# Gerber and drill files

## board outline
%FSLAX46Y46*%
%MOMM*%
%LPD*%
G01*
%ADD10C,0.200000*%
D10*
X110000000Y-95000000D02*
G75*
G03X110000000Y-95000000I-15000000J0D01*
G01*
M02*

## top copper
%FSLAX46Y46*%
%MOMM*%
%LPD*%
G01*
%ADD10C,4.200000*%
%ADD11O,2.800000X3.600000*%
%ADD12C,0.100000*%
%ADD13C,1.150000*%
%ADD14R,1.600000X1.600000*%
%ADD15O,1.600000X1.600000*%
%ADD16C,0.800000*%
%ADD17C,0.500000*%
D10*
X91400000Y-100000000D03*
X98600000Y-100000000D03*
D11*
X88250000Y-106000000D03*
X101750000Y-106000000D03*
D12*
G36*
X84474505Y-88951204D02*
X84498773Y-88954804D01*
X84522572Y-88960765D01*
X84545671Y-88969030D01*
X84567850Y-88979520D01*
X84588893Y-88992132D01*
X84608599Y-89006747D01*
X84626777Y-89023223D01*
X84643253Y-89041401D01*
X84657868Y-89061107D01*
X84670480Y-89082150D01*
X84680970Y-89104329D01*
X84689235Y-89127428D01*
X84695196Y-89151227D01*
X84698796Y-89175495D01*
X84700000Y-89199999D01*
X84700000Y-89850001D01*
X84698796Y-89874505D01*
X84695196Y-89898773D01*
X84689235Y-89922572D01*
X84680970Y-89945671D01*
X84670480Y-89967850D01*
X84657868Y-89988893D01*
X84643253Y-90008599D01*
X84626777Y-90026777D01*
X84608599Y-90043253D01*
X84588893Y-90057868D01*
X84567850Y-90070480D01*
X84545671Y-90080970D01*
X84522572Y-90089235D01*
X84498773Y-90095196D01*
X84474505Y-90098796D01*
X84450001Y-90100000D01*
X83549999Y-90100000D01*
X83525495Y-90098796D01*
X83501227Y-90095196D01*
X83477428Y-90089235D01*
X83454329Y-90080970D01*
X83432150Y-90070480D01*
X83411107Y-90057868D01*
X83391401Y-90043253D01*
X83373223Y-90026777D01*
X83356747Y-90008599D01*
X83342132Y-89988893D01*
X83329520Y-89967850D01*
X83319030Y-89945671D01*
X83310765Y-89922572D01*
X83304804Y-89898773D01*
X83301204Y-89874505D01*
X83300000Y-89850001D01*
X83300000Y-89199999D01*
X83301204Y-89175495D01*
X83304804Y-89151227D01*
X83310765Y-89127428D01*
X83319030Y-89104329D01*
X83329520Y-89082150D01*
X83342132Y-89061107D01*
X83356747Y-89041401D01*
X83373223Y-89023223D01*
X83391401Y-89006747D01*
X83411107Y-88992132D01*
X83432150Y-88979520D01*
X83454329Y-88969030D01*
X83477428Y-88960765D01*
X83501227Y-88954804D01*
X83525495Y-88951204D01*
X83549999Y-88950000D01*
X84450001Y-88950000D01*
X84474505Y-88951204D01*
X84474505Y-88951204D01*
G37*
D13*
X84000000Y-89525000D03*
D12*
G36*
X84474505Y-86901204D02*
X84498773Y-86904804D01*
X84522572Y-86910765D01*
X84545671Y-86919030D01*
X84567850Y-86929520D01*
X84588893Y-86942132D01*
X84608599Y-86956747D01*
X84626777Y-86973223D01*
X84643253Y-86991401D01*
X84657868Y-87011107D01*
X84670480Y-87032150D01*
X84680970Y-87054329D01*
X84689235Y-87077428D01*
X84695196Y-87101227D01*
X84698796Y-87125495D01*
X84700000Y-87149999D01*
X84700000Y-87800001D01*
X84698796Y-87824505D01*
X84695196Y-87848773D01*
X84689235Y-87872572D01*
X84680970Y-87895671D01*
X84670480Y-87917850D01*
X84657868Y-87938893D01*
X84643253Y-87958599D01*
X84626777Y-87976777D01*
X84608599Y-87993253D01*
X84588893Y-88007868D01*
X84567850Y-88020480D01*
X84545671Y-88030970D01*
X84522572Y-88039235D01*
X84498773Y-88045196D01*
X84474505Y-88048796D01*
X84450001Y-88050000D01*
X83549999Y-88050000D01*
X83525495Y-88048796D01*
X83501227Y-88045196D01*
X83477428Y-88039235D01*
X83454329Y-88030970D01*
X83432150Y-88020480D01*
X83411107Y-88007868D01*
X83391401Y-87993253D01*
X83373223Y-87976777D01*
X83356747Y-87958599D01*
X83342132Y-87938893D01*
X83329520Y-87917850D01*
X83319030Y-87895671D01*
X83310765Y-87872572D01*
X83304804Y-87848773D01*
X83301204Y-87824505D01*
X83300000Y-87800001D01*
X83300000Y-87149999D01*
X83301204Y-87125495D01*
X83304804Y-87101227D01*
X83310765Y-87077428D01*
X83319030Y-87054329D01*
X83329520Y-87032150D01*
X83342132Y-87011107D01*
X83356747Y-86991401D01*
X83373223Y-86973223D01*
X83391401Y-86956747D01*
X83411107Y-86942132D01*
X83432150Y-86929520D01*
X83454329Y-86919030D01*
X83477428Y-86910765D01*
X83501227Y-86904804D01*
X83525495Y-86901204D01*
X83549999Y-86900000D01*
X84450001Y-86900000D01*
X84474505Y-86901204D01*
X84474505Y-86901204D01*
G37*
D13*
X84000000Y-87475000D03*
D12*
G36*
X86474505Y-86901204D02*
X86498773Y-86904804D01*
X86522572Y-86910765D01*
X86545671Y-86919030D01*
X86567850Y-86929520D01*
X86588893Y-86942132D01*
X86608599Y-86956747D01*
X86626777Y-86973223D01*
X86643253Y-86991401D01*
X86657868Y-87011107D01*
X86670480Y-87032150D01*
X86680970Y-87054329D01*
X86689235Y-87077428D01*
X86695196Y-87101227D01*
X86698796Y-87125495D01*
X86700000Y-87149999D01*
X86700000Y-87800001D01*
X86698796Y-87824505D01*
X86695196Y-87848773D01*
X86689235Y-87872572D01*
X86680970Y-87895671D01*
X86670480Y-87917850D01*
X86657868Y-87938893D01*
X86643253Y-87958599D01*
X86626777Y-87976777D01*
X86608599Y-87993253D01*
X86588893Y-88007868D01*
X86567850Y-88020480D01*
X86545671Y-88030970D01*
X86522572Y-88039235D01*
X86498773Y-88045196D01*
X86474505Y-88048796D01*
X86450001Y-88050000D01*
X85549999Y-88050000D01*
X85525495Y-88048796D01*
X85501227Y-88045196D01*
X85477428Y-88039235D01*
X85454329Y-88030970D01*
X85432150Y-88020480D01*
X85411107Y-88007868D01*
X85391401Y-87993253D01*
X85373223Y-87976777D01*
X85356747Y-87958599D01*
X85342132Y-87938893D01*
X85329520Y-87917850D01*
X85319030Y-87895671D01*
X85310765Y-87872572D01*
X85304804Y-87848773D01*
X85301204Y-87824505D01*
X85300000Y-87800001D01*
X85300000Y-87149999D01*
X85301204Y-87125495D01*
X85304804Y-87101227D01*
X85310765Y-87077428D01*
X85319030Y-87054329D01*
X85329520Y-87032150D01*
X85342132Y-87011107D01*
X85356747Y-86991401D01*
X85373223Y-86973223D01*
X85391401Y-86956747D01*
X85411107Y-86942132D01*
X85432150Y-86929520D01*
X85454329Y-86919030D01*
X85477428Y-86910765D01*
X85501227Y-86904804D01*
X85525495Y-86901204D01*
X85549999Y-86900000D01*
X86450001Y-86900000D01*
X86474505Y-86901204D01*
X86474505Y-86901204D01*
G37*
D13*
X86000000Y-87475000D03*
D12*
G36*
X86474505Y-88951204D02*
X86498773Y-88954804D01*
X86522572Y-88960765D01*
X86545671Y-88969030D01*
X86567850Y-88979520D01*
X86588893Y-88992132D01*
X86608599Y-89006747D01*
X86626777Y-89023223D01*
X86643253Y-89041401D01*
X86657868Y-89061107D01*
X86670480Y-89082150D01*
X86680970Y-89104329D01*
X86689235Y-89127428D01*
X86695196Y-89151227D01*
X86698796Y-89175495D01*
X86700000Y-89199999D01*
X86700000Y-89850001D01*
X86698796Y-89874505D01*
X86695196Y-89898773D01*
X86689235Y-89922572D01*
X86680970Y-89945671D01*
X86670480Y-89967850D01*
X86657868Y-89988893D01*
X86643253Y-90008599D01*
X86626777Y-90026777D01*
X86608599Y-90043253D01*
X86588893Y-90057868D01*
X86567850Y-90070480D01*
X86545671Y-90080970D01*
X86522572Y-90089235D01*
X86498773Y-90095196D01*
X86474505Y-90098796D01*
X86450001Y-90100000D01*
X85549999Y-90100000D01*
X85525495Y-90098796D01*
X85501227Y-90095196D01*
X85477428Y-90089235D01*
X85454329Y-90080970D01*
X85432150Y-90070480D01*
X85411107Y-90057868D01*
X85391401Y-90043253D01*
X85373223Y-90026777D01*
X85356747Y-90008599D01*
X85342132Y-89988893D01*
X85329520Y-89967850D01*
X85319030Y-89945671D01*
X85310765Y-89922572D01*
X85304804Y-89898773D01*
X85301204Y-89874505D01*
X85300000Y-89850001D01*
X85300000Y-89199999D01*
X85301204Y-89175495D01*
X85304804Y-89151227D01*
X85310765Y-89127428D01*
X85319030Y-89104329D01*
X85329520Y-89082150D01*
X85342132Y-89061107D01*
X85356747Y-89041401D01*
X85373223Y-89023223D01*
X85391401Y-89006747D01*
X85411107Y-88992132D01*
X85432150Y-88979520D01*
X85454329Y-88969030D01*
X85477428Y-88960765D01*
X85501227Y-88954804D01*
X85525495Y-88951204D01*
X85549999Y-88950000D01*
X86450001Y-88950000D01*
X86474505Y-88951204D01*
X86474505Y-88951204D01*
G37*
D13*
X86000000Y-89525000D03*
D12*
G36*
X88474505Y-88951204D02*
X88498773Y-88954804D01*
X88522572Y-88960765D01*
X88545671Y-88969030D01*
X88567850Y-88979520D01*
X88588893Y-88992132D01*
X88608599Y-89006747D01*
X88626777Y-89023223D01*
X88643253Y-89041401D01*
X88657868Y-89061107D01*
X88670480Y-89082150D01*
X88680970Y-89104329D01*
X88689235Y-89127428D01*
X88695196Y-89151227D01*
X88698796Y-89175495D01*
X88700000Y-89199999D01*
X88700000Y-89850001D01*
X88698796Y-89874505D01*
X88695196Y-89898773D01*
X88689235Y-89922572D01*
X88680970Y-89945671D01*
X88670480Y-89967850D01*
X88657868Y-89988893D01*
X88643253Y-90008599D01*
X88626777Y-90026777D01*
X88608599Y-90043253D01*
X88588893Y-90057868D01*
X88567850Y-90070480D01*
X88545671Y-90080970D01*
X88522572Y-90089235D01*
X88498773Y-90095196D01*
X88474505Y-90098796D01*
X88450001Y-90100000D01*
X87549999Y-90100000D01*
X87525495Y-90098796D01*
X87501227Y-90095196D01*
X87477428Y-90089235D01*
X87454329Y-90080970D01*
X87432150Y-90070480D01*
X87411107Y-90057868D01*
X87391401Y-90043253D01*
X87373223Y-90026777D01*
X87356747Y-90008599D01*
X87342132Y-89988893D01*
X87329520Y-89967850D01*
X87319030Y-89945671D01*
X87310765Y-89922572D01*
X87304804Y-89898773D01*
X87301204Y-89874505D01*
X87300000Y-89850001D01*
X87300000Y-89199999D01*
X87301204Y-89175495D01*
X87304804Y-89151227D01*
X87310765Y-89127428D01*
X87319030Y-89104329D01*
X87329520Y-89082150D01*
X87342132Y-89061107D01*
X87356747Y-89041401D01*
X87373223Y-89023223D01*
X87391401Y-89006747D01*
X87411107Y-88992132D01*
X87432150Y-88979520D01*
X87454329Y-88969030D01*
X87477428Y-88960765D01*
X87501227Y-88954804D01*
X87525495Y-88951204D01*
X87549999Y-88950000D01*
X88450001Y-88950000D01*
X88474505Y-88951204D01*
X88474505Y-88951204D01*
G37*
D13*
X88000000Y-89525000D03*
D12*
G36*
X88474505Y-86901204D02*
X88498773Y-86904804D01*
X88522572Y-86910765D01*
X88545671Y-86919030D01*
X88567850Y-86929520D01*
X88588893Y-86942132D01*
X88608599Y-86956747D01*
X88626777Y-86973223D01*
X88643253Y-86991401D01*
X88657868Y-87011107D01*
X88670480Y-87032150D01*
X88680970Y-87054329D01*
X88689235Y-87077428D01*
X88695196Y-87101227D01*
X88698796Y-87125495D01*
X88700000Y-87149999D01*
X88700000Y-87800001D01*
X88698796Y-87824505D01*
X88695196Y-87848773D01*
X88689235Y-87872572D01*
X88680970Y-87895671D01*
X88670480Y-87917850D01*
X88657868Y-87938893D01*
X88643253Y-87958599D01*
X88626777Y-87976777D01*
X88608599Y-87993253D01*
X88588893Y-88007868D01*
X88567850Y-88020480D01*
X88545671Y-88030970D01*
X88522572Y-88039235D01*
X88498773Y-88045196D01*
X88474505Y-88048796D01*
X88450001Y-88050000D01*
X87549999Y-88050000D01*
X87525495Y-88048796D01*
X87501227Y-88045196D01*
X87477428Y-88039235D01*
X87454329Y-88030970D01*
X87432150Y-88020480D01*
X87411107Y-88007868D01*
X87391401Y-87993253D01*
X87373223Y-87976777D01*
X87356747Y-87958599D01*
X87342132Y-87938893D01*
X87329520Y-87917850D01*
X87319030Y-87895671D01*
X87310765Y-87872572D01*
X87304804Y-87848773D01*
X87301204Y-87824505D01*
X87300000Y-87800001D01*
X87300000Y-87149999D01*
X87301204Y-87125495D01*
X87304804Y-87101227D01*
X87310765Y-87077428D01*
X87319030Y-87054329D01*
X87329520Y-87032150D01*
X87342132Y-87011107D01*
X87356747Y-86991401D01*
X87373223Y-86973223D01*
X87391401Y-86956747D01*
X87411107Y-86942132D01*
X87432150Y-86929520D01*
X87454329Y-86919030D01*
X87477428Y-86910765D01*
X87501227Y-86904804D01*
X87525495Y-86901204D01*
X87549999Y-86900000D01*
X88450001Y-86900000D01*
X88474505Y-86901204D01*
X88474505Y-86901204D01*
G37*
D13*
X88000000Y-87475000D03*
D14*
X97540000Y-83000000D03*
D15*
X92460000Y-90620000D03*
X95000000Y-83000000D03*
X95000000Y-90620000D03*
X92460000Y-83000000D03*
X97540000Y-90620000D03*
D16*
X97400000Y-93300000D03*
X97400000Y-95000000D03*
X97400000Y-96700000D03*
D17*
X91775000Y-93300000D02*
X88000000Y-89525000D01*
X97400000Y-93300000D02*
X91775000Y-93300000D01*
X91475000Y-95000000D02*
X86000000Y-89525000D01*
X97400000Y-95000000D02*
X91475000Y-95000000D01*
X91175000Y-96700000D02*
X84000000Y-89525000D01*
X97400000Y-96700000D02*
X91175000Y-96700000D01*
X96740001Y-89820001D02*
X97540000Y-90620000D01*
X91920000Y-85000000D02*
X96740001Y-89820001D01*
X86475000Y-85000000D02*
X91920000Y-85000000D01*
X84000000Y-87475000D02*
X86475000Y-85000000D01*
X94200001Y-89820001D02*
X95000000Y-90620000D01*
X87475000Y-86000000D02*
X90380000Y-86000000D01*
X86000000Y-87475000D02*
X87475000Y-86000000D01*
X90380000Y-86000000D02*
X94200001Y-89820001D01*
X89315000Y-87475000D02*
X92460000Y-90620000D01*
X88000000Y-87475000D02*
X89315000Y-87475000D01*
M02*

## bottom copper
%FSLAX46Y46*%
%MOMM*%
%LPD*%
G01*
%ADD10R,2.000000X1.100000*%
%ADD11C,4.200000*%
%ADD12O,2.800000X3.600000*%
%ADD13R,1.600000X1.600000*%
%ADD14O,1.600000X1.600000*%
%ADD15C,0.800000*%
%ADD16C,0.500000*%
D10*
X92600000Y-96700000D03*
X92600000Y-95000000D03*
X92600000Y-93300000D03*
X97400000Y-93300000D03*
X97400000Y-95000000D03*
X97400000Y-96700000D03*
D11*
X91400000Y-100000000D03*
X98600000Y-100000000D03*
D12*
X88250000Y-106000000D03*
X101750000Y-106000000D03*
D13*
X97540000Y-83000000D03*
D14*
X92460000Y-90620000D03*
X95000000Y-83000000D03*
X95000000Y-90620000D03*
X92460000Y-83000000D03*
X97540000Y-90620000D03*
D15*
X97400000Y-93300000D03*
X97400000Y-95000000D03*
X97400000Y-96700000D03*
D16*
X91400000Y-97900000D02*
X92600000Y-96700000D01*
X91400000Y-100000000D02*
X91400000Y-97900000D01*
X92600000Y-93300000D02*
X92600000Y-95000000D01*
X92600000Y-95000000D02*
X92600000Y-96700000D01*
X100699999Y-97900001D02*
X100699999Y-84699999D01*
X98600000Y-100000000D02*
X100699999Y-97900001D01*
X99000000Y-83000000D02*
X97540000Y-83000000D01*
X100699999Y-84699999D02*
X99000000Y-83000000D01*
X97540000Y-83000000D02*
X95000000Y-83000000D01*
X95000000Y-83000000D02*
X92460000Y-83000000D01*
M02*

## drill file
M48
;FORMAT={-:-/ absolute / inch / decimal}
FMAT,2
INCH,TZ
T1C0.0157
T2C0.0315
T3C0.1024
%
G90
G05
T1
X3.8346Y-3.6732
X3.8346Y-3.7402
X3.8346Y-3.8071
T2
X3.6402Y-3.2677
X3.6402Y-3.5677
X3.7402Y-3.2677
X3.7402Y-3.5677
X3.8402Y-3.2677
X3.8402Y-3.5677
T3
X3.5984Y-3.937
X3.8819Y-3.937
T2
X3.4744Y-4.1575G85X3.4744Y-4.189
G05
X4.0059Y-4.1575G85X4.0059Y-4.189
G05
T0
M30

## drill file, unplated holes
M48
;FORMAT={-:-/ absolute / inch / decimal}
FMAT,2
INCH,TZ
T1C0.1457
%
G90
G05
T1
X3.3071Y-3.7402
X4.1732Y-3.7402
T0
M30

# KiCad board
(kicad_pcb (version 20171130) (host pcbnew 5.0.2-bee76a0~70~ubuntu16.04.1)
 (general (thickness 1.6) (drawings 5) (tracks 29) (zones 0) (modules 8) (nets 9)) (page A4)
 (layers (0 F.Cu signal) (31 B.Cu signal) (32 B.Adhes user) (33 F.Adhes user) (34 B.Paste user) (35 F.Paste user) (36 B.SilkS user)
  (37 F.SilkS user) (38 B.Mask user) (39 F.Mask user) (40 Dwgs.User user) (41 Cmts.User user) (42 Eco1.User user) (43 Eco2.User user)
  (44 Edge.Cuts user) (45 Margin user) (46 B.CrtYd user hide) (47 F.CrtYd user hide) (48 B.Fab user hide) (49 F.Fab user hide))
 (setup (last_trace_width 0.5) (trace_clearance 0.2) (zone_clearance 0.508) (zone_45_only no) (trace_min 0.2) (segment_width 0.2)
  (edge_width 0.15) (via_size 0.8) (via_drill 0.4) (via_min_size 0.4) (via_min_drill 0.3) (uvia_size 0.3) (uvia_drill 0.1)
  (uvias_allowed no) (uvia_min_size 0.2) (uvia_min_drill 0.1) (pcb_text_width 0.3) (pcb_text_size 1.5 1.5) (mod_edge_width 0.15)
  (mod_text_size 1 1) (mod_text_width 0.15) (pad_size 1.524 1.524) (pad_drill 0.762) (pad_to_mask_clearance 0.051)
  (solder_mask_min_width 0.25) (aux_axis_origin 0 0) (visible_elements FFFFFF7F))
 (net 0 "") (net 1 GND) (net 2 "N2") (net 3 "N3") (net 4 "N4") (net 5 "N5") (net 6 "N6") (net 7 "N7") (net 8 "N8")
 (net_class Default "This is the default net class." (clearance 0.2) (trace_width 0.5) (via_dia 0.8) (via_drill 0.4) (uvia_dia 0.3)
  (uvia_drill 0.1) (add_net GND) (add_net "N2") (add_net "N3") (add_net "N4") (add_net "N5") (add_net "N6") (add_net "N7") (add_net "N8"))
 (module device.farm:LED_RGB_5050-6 (layer B.Cu) (at 95 95)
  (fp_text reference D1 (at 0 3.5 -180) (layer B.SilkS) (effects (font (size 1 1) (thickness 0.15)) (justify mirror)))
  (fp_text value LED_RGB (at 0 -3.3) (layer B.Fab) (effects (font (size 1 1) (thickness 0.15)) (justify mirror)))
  (pad 1 smd rect (at -2.4 1.7 270) (size 1.1 2) (layers B.Cu B.Paste B.Mask) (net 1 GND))
  (pad 2 smd rect (at -2.4 0 270) (size 1.1 2) (layers B.Cu B.Paste B.Mask) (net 1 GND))
  (pad 3 smd rect (at -2.4 -1.7 270) (size 1.1 2) (layers B.Cu B.Paste B.Mask) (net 1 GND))
  (pad 4 smd rect (at 2.4 -1.7 270) (size 1.1 2) (layers B.Cu B.Paste B.Mask) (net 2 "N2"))
  (pad 5 smd rect (at 2.4 0 270) (size 1.1 2) (layers B.Cu B.Paste B.Mask) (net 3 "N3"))
  (pad 6 smd rect (at 2.4 1.7 270) (size 1.1 2) (layers B.Cu B.Paste B.Mask) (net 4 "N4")))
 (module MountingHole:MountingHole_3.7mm (layer F.Cu) (at 84 95)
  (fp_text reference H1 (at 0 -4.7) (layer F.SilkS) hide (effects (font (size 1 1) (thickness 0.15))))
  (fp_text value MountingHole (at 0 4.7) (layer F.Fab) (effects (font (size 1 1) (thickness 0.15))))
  (pad 1 np_thru_hole circle (at 0 0) (size 3.7 3.7) (drill 3.7) (layers *.Cu *.Mask)))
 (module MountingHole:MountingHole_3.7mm (layer F.Cu) (at 106 95)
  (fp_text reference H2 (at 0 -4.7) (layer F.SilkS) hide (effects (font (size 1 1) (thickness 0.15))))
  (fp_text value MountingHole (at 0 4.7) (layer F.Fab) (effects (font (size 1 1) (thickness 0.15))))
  (pad 1 np_thru_hole circle (at 0 0) (size 3.7 3.7) (drill 3.7) (layers *.Cu *.Mask)))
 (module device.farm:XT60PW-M (layer F.Cu) (at 95 100)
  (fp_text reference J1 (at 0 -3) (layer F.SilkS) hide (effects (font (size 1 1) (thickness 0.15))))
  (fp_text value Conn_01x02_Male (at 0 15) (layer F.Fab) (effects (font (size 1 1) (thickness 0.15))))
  (pad 1 thru_hole circle (at -3.6 0) (size 4.2 4.2) (drill 2.6) (layers *.Cu *.Mask) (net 1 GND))
  (pad 2 thru_hole circle (at 3.6 0) (size 4.2 4.2) (drill 2.6) (layers *.Cu *.Mask) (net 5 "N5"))
  (pad "" thru_hole oval (at -6.75 6) (size 2.8 3.6) (drill oval 0.8 1.6) (layers *.Cu *.Mask))
  (pad "" thru_hole oval (at 6.75 6) (size 2.8 3.6) (drill oval 0.8 1.6) (layers *.Cu *.Mask)))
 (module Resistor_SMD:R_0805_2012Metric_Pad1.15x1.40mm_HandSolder (layer F.Cu) (at 84 88.5 90)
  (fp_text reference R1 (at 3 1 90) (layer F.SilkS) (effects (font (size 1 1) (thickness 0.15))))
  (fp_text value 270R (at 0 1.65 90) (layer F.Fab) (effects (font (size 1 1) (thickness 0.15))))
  (pad 1 smd roundrect (at -1.025 0 90) (size 1.15 1.4) (layers F.Cu F.Paste F.Mask) (roundrect_rratio 0.217391) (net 4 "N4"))
  (pad 2 smd roundrect (at 1.025 0 90) (size 1.15 1.4) (layers F.Cu F.Paste F.Mask) (roundrect_rratio 0.217391) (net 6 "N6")))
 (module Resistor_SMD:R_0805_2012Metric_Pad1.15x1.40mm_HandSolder (layer F.Cu) (at 86 88.5 90)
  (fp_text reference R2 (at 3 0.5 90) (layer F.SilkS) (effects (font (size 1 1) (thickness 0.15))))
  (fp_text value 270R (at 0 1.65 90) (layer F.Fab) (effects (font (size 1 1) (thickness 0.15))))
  (pad 2 smd roundrect (at 1.025 0 90) (size 1.15 1.4) (layers F.Cu F.Paste F.Mask) (roundrect_rratio 0.217391) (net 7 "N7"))
  (pad 1 smd roundrect (at -1.025 0 90) (size 1.15 1.4) (layers F.Cu F.Paste F.Mask) (roundrect_rratio 0.217391) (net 3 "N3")))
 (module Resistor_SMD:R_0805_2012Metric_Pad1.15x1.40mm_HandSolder (layer F.Cu) (at 88 88.5 90)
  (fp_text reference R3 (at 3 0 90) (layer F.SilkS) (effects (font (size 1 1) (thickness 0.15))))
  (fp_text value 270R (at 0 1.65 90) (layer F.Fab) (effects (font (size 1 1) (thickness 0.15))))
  (pad 1 smd roundrect (at -1.025 0 90) (size 1.15 1.4) (layers F.Cu F.Paste F.Mask) (roundrect_rratio 0.217391) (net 2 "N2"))
  (pad 2 smd roundrect (at 1.025 0 90) (size 1.15 1.4) (layers F.Cu F.Paste F.Mask) (roundrect_rratio 0.217391) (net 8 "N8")))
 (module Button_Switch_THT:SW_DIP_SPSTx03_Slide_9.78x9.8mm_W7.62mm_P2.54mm (layer F.Cu) (at 97.54 83 270)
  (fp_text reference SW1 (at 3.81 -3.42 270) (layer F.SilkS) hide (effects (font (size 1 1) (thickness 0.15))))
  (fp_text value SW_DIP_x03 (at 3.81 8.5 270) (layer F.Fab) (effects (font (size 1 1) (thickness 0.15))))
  (pad 1 thru_hole rect (at 0 0 270) (size 1.6 1.6) (drill 0.8) (layers *.Cu *.Mask) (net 5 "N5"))
  (pad 4 thru_hole oval (at 7.62 5.08 270) (size 1.6 1.6) (drill 0.8) (layers *.Cu *.Mask) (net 8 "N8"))
  (pad 2 thru_hole oval (at 0 2.54 270) (size 1.6 1.6) (drill 0.8) (layers *.Cu *.Mask) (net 5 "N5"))
  (pad 5 thru_hole oval (at 7.62 2.54 270) (size 1.6 1.6) (drill 0.8) (layers *.Cu *.Mask) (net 7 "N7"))
  (pad 3 thru_hole oval (at 0 5.08 270) (size 1.6 1.6) (drill 0.8) (layers *.Cu *.Mask) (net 5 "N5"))
  (pad 6 thru_hole oval (at 7.62 0 270) (size 1.6 1.6) (drill 0.8) (layers *.Cu *.Mask) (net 6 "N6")))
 (gr_circle (center 95 95) (end 110 95) (layer Edge.Cuts) (width 0.2))
 (segment (start 91.4 97.9) (end 92.6 96.7) (width 0.5) (layer B.Cu) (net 1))
 (segment (start 91.4 100) (end 91.4 97.9) (width 0.5) (layer B.Cu) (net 1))
 (segment (start 92.6 93.3) (end 92.6 95) (width 0.5) (layer B.Cu) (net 1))
 (segment (start 92.6 95) (end 92.6 96.7) (width 0.5) (layer B.Cu) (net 1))
 (via (at 97.4 93.3) (size 0.8) (drill 0.4) (layers F.Cu B.Cu) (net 2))
 (segment (start 91.775 93.3) (end 88 89.525) (width 0.5) (layer F.Cu) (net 2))
 (segment (start 97.4 93.3) (end 91.775 93.3) (width 0.5) (layer F.Cu) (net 2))
 (via (at 97.4 95) (size 0.8) (drill 0.4) (layers F.Cu B.Cu) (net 3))
 (segment (start 91.475 95) (end 86 89.525) (width 0.5) (layer F.Cu) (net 3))
 (segment (start 97.4 95) (end 91.475 95) (width 0.5) (layer F.Cu) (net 3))
 (via (at 97.4 96.7) (size 0.8) (drill 0.4) (layers F.Cu B.Cu) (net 4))
 (segment (start 91.175 96.7) (end 84 89.525) (width 0.5) (layer F.Cu) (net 4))
 (segment (start 97.4 96.7) (end 91.175 96.7) (width 0.5) (layer F.Cu) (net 4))
 (segment (start 100.699999 97.900001) (end 100.699999 84.699999) (width 0.5) (layer B.Cu) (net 5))
 (segment (start 98.6 100) (end 100.699999 97.900001) (width 0.5) (layer B.Cu) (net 5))
 (segment (start 99 83) (end 97.54 83) (width 0.5) (layer B.Cu) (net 5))
 (segment (start 100.699999 84.699999) (end 99 83) (width 0.5) (layer B.Cu) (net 5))
 (segment (start 97.54 83) (end 95 83) (width 0.5) (layer B.Cu) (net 5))
 (segment (start 95 83) (end 92.46 83) (width 0.5) (layer B.Cu) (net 5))
 (segment (start 96.740001 89.820001) (end 97.54 90.62) (width 0.5) (layer F.Cu) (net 6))
 (segment (start 91.92 85) (end 96.740001 89.820001) (width 0.5) (layer F.Cu) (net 6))
 (segment (start 86.475 85) (end 91.92 85) (width 0.5) (layer F.Cu) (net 6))
 (segment (start 84 87.475) (end 86.475 85) (width 0.5) (layer F.Cu) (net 6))
 (segment (start 94.200001 89.820001) (end 95 90.62) (width 0.5) (layer F.Cu) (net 7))
 (segment (start 87.475 86) (end 90.38 86) (width 0.5) (layer F.Cu) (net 7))
 (segment (start 86 87.475) (end 87.475 86) (width 0.5) (layer F.Cu) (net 7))
 (segment (start 90.38 86) (end 94.200001 89.820001) (width 0.5) (layer F.Cu) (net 7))
 (segment (start 89.315 87.475) (end 92.46 90.62) (width 0.5) (layer F.Cu) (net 8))
 (segment (start 88 87.475) (end 89.315 87.475) (width 0.5) (layer F.Cu) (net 8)))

